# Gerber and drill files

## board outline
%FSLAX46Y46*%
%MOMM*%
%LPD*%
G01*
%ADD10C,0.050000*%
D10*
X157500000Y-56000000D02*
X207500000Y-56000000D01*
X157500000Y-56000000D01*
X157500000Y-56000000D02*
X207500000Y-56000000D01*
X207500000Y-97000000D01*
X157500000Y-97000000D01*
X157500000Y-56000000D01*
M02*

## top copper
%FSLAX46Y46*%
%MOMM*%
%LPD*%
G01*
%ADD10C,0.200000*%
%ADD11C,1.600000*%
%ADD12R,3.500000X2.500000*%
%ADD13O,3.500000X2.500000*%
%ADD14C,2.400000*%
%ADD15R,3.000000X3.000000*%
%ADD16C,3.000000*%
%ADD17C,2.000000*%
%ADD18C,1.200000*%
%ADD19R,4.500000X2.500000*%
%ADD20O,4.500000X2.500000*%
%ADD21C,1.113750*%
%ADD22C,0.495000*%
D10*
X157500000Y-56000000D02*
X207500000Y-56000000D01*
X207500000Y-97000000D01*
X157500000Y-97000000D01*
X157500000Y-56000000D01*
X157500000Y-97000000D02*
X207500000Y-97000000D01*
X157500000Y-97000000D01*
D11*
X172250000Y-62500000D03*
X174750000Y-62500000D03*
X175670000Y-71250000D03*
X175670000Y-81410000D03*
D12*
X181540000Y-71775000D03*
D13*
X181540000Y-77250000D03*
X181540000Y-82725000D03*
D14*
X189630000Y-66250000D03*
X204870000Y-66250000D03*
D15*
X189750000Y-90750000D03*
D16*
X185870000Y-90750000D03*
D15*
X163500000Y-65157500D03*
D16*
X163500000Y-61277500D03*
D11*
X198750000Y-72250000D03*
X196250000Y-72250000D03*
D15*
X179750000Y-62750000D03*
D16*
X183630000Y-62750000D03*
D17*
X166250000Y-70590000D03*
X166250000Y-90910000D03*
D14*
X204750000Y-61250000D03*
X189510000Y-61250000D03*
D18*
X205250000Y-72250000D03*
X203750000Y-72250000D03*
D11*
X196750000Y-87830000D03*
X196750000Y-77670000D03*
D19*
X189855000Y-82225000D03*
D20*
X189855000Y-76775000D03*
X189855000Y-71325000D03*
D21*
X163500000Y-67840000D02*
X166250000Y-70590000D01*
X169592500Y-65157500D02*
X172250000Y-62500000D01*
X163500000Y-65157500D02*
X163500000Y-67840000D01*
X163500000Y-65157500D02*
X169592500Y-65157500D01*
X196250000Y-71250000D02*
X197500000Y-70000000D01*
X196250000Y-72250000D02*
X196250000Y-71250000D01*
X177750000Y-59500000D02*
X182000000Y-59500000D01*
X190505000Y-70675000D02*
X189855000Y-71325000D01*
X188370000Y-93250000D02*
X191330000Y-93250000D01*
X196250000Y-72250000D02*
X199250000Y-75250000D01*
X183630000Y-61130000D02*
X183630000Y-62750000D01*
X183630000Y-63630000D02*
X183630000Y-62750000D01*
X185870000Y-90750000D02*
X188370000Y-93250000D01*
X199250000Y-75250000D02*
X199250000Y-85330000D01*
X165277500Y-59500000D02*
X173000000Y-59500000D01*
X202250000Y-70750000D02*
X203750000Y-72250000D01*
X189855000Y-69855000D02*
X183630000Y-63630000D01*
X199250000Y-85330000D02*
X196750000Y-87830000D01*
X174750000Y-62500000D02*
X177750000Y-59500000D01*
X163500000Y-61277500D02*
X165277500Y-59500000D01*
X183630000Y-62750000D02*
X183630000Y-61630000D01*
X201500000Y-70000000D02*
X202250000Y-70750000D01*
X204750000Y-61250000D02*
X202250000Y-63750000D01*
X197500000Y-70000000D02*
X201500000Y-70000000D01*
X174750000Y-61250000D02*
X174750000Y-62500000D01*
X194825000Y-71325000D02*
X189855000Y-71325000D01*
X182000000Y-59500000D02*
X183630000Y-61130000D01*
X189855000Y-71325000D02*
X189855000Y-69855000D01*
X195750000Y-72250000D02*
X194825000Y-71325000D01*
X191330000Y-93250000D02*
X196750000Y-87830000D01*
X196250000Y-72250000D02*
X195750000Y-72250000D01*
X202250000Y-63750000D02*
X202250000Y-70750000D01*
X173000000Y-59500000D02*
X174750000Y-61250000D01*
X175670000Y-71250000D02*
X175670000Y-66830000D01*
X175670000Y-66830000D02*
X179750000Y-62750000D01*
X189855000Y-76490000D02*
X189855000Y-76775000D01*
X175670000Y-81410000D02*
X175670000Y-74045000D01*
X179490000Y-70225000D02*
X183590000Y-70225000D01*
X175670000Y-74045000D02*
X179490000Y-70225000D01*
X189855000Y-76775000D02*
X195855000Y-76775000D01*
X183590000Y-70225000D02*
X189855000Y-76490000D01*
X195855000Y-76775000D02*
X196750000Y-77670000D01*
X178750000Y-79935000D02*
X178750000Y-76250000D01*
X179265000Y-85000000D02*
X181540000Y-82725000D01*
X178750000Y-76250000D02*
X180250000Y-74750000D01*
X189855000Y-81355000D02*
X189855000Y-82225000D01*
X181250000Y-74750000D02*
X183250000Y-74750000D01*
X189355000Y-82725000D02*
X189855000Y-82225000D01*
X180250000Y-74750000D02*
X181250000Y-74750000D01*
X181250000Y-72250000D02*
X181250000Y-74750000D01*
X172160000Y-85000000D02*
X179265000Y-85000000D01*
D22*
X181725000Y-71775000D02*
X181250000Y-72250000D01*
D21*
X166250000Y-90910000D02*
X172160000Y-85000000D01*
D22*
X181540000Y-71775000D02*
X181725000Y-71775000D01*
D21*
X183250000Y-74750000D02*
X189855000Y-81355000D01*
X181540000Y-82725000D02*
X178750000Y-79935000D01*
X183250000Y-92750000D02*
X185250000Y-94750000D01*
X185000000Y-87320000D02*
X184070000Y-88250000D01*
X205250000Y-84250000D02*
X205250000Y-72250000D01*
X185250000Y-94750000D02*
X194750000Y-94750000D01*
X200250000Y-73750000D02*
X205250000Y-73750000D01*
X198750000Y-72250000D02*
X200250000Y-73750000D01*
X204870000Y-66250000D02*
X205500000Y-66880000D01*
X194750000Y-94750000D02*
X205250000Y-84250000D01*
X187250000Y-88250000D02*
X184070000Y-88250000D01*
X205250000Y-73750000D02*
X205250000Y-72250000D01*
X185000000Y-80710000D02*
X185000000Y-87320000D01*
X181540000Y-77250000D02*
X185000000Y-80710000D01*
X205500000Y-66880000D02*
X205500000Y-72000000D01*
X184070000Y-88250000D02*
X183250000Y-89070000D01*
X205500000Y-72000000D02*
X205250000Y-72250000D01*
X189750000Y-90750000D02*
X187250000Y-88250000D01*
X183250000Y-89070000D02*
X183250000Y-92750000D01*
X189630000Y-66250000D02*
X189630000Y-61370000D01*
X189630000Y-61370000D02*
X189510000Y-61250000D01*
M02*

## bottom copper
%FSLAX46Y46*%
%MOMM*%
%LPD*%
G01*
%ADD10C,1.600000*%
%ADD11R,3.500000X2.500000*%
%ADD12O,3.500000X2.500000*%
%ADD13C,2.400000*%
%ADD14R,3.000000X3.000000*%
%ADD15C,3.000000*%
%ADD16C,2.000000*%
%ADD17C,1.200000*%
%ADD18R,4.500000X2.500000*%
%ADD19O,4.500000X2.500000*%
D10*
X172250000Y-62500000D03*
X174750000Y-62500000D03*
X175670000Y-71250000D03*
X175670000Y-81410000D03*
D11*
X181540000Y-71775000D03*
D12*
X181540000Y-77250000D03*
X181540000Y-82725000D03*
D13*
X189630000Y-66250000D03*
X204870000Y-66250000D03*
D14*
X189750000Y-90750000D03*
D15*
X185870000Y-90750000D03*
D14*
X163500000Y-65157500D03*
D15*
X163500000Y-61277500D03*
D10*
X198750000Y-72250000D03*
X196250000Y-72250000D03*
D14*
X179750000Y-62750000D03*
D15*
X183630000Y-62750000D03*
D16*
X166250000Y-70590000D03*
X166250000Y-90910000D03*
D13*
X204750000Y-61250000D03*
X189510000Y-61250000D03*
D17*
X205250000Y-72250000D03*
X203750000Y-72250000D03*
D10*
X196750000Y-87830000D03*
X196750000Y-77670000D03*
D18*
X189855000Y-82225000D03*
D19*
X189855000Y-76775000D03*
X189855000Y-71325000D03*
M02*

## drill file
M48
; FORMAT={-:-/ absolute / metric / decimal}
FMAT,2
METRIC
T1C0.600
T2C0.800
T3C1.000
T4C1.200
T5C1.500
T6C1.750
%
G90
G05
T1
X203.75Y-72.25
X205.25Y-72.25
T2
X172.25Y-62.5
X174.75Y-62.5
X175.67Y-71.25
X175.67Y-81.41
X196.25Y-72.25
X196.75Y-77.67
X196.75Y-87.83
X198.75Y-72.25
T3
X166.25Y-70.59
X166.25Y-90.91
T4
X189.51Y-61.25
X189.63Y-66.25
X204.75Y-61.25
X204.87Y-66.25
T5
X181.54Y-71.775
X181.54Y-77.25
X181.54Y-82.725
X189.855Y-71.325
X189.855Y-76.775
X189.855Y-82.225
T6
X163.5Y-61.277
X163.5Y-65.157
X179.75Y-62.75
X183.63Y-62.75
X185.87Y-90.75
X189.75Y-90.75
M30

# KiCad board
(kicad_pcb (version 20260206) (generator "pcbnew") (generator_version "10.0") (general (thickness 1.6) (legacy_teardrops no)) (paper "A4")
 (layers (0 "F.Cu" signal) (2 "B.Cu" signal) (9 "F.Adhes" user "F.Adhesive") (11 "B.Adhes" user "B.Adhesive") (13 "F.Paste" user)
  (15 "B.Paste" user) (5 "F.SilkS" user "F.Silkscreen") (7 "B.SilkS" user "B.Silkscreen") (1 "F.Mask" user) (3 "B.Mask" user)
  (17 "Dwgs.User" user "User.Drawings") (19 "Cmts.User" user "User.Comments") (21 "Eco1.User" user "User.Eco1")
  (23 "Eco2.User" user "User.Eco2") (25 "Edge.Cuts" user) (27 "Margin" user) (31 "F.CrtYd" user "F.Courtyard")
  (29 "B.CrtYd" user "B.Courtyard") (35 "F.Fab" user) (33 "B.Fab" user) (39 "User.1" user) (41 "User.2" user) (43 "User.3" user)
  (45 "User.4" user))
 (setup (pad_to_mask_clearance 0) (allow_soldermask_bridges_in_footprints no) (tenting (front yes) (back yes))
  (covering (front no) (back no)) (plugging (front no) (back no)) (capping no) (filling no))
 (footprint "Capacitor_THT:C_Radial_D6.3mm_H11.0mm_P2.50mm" (layer "F.Cu") (at 172.25 62.5)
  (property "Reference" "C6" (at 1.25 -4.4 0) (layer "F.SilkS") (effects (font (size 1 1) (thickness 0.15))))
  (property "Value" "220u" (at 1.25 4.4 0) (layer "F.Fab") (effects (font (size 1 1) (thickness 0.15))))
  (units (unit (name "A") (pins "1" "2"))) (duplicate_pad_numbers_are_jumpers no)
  (pad "1" thru_hole circle (at 0 0) (size 1.6 1.6) (drill 0.8) (layers "*.Cu" "*.Mask") (remove_unused_layers no) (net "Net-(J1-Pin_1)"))
  (pad "2" thru_hole circle (at 2.5 0) (size 1.6 1.6) (drill 0.8) (layers "*.Cu" "*.Mask") (remove_unused_layers no) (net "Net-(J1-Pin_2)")))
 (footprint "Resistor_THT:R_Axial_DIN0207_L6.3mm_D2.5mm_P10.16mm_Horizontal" (layer "F.Cu") (at 175.67 71.25 -90)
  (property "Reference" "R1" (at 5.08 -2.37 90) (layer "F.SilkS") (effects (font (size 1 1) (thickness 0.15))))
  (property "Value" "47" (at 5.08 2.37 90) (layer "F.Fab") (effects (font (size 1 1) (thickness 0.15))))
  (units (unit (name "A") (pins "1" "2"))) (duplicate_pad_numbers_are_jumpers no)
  (pad "1" thru_hole circle (at 0 0 270) (size 1.6 1.6) (drill 0.8) (layers "*.Cu" "*.Mask") (remove_unused_layers no)
   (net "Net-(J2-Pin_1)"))
  (pad "2" thru_hole circle (at 10.16 0 270) (size 1.6 1.6) (drill 0.8) (layers "*.Cu" "*.Mask") (remove_unused_layers no)
   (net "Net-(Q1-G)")))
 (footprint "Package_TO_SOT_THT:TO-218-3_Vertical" (layer "F.Cu") (at 181.54 71.775 -90)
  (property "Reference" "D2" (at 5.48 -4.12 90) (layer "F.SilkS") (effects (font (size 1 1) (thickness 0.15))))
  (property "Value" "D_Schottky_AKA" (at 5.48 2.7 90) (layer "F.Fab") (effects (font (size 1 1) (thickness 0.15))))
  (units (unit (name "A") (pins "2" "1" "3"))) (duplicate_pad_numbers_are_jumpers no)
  (pad "1" thru_hole rect (at 0 0 270) (size 2.5 3.5) (drill 1.5) (layers "*.Cu" "*.Mask") (remove_unused_layers no) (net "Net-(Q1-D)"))
  (pad "2" thru_hole oval (at 5.475 0 270) (size 2.5 3.5) (drill 1.5) (layers "*.Cu" "*.Mask") (remove_unused_layers no) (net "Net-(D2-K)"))
  (pad "3" thru_hole oval (at 10.95 0 270) (size 2.5 3.5) (drill 1.5) (layers "*.Cu" "*.Mask") (remove_unused_layers no) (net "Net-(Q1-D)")))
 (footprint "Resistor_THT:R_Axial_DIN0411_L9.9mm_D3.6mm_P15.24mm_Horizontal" (layer "F.Cu") (at 189.63 66.25)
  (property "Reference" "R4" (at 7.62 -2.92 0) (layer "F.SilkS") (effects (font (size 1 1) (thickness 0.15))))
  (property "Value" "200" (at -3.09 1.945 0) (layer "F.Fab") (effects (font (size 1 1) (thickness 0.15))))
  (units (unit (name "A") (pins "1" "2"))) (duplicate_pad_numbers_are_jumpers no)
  (pad "1" thru_hole circle (at 0 0) (size 2.4 2.4) (drill 1.2) (layers "*.Cu" "*.Mask") (remove_unused_layers no) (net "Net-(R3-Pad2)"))
  (pad "2" thru_hole circle (at 15.24 0) (size 2.4 2.4) (drill 1.2) (layers "*.Cu" "*.Mask") (remove_unused_layers no) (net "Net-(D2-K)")))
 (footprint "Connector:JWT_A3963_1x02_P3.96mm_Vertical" (layer "F.Cu") (at 189.75 90.75 180)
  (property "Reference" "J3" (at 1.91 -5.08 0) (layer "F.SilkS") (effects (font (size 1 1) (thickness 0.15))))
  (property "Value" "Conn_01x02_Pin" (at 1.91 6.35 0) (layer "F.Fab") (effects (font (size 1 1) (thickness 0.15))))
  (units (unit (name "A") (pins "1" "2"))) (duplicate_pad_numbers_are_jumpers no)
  (pad "1" thru_hole rect (at 0 0 180) (size 3 3) (drill 1.75) (layers "*.Cu" "*.Mask") (remove_unused_layers no) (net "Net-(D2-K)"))
  (pad "2" thru_hole circle (at 3.88 0 180) (size 3 3) (drill 1.75) (layers "*.Cu" "*.Mask") (remove_unused_layers no)
   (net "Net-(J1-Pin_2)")))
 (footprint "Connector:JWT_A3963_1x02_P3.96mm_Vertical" (layer "F.Cu") (at 163.5 65.1575 90)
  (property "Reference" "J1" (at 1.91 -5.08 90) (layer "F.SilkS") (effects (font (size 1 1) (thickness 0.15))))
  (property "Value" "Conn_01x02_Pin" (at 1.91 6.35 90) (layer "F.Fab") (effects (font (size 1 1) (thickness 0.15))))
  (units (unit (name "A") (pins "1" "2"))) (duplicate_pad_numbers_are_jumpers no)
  (pad "1" thru_hole rect (at 0 0 90) (size 3 3) (drill 1.75) (layers "*.Cu" "*.Mask") (remove_unused_layers no) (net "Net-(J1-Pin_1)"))
  (pad "2" thru_hole circle (at 3.88 0 90) (size 3 3) (drill 1.75) (layers "*.Cu" "*.Mask") (remove_unused_layers no) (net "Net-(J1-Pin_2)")))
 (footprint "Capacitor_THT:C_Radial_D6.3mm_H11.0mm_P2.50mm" (layer "F.Cu") (at 198.75 72.25 180)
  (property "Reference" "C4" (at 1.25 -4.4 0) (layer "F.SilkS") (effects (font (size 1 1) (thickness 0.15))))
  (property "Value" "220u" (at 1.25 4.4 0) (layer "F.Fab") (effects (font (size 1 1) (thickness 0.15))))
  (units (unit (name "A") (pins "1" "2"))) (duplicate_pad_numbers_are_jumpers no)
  (pad "1" thru_hole circle (at 0 0 180) (size 1.6 1.6) (drill 0.8) (layers "*.Cu" "*.Mask") (remove_unused_layers no) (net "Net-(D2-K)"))
  (pad "2" thru_hole circle (at 2.5 0 180) (size 1.6 1.6) (drill 0.8) (layers "*.Cu" "*.Mask") (remove_unused_layers no)
   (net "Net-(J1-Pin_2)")))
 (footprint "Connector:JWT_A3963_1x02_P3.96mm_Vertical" (layer "F.Cu") (at 179.75 62.75)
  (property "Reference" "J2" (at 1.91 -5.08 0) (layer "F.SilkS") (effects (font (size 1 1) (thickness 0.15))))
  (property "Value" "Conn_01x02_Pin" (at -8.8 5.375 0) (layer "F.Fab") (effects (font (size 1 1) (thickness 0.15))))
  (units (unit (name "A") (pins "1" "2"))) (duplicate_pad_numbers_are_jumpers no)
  (pad "1" thru_hole rect (at 0 0) (size 3 3) (drill 1.75) (layers "*.Cu" "*.Mask") (remove_unused_layers no) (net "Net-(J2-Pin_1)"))
  (pad "2" thru_hole circle (at 3.88 0) (size 3 3) (drill 1.75) (layers "*.Cu" "*.Mask") (remove_unused_layers no) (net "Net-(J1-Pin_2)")))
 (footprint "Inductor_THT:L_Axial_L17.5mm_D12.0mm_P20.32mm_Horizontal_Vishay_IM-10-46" (layer "F.Cu") (at 166.25 70.59 -90)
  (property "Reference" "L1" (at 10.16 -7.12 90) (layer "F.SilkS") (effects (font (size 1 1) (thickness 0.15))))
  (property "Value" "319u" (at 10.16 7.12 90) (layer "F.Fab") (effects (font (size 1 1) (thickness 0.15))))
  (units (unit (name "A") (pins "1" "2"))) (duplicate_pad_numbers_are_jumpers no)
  (pad "1" thru_hole circle (at 0 0 270) (size 2 2) (drill 1) (layers "*.Cu" "*.Mask") (remove_unused_layers no) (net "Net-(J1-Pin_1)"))
  (pad "2" thru_hole circle (at 20.32 0 270) (size 2 2) (drill 1) (layers "*.Cu" "*.Mask") (remove_unused_layers no) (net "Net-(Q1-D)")))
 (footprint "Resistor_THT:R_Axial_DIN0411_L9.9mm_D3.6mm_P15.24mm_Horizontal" (layer "F.Cu") (at 204.75 61.25 180)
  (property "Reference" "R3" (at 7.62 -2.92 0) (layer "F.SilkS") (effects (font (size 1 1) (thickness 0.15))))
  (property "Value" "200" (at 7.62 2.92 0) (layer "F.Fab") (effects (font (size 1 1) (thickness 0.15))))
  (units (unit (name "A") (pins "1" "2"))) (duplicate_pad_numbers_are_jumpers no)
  (pad "1" thru_hole circle (at 0 0 180) (size 2.4 2.4) (drill 1.2) (layers "*.Cu" "*.Mask") (remove_unused_layers no)
   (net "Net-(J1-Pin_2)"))
  (pad "2" thru_hole circle (at 15.24 0 180) (size 2.4 2.4) (drill 1.2) (layers "*.Cu" "*.Mask") (remove_unused_layers no)
   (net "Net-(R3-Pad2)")))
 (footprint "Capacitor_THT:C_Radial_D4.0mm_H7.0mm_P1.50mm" (layer "F.Cu") (at 205.25 72.25 180)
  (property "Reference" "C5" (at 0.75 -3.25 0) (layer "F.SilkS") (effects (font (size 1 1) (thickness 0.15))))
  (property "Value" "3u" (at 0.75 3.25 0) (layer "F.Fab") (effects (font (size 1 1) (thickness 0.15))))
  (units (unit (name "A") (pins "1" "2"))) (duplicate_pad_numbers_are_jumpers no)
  (pad "1" thru_hole circle (at 0 0 180) (size 1.2 1.2) (drill 0.6) (layers "*.Cu" "*.Mask") (remove_unused_layers no) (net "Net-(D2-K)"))
  (pad "2" thru_hole circle (at 1.5 0 180) (size 1.2 1.2) (drill 0.6) (layers "*.Cu" "*.Mask") (remove_unused_layers no)
   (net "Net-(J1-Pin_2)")))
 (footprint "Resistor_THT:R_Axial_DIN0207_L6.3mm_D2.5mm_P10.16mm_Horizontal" (layer "F.Cu") (at 196.75 87.83 90)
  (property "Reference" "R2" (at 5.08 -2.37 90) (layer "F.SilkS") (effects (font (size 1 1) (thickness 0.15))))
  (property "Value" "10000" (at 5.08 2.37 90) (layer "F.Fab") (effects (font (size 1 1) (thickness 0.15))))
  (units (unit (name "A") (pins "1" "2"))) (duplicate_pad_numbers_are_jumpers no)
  (pad "1" thru_hole circle (at 0 0 90) (size 1.6 1.6) (drill 0.8) (layers "*.Cu" "*.Mask") (remove_unused_layers no) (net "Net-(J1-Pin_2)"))
  (pad "2" thru_hole circle (at 10.16 0 90) (size 1.6 1.6) (drill 0.8) (layers "*.Cu" "*.Mask") (remove_unused_layers no) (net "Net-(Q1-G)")))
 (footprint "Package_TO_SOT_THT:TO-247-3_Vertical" (layer "B.Cu") (at 189.855 82.225 90)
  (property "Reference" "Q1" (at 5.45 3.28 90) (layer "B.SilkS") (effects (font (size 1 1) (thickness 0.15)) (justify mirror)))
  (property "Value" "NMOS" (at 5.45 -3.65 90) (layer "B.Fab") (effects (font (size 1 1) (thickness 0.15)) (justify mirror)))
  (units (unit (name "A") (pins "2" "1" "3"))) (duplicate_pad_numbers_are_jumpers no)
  (pad "1" thru_hole rect (at 0 0 90) (size 2.5 4.5) (drill 1.5) (layers "*.Cu" "*.Mask") (remove_unused_layers no) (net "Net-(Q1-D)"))
  (pad "2" thru_hole oval (at 5.45 0 90) (size 2.5 4.5) (drill 1.5) (layers "*.Cu" "*.Mask") (remove_unused_layers no) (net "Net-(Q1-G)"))
  (pad "3" thru_hole oval (at 10.9 0 90) (size 2.5 4.5) (drill 1.5) (layers "*.Cu" "*.Mask") (remove_unused_layers no)
   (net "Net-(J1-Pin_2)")))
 (gr_rect (start 157.5 56) (end 207.5 97) (stroke (width 0.2) (type default)) (fill no) (layer "F.Cu"))
 (gr_rect (start 157.5 97) (end 207.5 97) (stroke (width 0.2) (type default)) (fill no) (layer "F.Cu"))
 (gr_rect (start 157.5 56) (end 207.5 56) (stroke (width 0.05) (type default)) (fill no) (layer "Edge.Cuts"))
 (gr_rect (start 157.5 56) (end 207.5 97) (stroke (width 0.05) (type default)) (fill no) (layer "Edge.Cuts"))
 (segment (start 163.5 67.84) (end 166.25 70.59) (width 1.11375) (layer "F.Cu") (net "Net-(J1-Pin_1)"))
 (segment (start 169.5925 65.1575) (end 172.25 62.5) (width 1.11375) (layer "F.Cu") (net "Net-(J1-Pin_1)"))
 (segment (start 163.5 65.1575) (end 163.5 67.84) (width 1.11375) (layer "F.Cu") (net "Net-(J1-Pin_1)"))
 (segment (start 163.5 65.1575) (end 169.5925 65.1575) (width 1.11375) (layer "F.Cu") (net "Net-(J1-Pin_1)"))
 (segment (start 196.25 71.25) (end 197.5 70) (width 1.11375) (layer "F.Cu") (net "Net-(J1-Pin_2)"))
 (segment (start 196.25 72.25) (end 196.25 71.25) (width 1.11375) (layer "F.Cu") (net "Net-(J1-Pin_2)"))
 (segment (start 177.75 59.5) (end 182 59.5) (width 1.11375) (layer "F.Cu") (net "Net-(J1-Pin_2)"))
 (segment (start 190.505 70.675) (end 189.855 71.325) (width 1.11375) (layer "F.Cu") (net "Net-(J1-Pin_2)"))
 (segment (start 188.37 93.25) (end 191.33 93.25) (width 1.11375) (layer "F.Cu") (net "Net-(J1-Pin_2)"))
 (segment (start 196.25 72.25) (end 199.25 75.25) (width 1.11375) (layer "F.Cu") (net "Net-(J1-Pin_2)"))
 (segment (start 183.63 61.13) (end 183.63 62.75) (width 1.11375) (layer "F.Cu") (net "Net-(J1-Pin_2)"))
 (segment (start 183.63 63.63) (end 183.63 62.75) (width 1.11375) (layer "F.Cu") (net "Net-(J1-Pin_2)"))
 (segment (start 185.87 90.75) (end 188.37 93.25) (width 1.11375) (layer "F.Cu") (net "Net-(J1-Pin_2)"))
 (segment (start 199.25 75.25) (end 199.25 85.33) (width 1.11375) (layer "F.Cu") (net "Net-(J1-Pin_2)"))
 (segment (start 165.2775 59.5) (end 173 59.5) (width 1.11375) (layer "F.Cu") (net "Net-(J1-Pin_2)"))
 (segment (start 202.25 70.75) (end 203.75 72.25) (width 1.11375) (layer "F.Cu") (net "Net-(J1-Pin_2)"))
 (segment (start 189.855 69.855) (end 183.63 63.63) (width 1.11375) (layer "F.Cu") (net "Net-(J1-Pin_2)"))
 (segment (start 199.25 85.33) (end 196.75 87.83) (width 1.11375) (layer "F.Cu") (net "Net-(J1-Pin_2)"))
 (segment (start 174.75 62.5) (end 177.75 59.5) (width 1.11375) (layer "F.Cu") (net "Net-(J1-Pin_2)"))
 (segment (start 163.5 61.2775) (end 165.2775 59.5) (width 1.11375) (layer "F.Cu") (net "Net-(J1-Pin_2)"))
 (segment (start 183.63 62.75) (end 183.63 61.63) (width 1.11375) (layer "F.Cu") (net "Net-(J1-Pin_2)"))
 (segment (start 201.5 70) (end 202.25 70.75) (width 1.11375) (layer "F.Cu") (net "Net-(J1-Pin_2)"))
 (segment (start 204.75 61.25) (end 202.25 63.75) (width 1.11375) (layer "F.Cu") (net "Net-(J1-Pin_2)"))
 (segment (start 197.5 70) (end 201.5 70) (width 1.11375) (layer "F.Cu") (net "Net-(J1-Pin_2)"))
 (segment (start 174.75 61.25) (end 174.75 62.5) (width 1.11375) (layer "F.Cu") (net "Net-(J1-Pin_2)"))
 (segment (start 194.825 71.325) (end 189.855 71.325) (width 1.11375) (layer "F.Cu") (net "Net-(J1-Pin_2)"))
 (segment (start 182 59.5) (end 183.63 61.13) (width 1.11375) (layer "F.Cu") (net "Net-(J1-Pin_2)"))
 (segment (start 189.855 71.325) (end 189.855 69.855) (width 1.11375) (layer "F.Cu") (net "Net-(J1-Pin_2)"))
 (segment (start 195.75 72.25) (end 194.825 71.325) (width 1.11375) (layer "F.Cu") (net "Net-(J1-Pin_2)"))
 (segment (start 191.33 93.25) (end 196.75 87.83) (width 1.11375) (layer "F.Cu") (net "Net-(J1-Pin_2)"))
 (segment (start 196.25 72.25) (end 195.75 72.25) (width 1.11375) (layer "F.Cu") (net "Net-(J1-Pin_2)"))
 (segment (start 202.25 63.75) (end 202.25 70.75) (width 1.11375) (layer "F.Cu") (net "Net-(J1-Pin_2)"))
 (segment (start 173 59.5) (end 174.75 61.25) (width 1.11375) (layer "F.Cu") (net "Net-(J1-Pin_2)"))
 (segment (start 175.67 71.25) (end 175.67 66.83) (width 1.11375) (layer "F.Cu") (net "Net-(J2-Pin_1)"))
 (segment (start 175.67 66.83) (end 179.75 62.75) (width 1.11375) (layer "F.Cu") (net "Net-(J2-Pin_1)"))
 (segment (start 189.855 76.49) (end 189.855 76.775) (width 1.11375) (layer "F.Cu") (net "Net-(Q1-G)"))
 (segment (start 175.67 81.41) (end 175.67 74.045) (width 1.11375) (layer "F.Cu") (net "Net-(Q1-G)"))
 (segment (start 179.49 70.225) (end 183.59 70.225) (width 1.11375) (layer "F.Cu") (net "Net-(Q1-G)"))
 (segment (start 175.67 74.045) (end 179.49 70.225) (width 1.11375) (layer "F.Cu") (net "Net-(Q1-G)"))
 (segment (start 189.855 76.775) (end 195.855 76.775) (width 1.11375) (layer "F.Cu") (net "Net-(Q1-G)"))
 (segment (start 183.59 70.225) (end 189.855 76.49) (width 1.11375) (layer "F.Cu") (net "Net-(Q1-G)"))
 (segment (start 195.855 76.775) (end 196.75 77.67) (width 1.11375) (layer "F.Cu") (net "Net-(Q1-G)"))
 (segment (start 178.75 79.935) (end 178.75 76.25) (width 1.11375) (layer "F.Cu") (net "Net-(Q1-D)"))
 (segment (start 179.265 85) (end 181.54 82.725) (width 1.11375) (layer "F.Cu") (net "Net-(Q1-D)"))
 (segment (start 178.75 76.25) (end 180.25 74.75) (width 1.11375) (layer "F.Cu") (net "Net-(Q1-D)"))
 (segment (start 189.855 81.355) (end 189.855 82.225) (width 1.11375) (layer "F.Cu") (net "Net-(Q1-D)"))
 (segment (start 181.25 74.75) (end 183.25 74.75) (width 1.11375) (layer "F.Cu") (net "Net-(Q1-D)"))
 (segment (start 189.355 82.725) (end 189.855 82.225) (width 1.11375) (layer "F.Cu") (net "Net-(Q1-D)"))
 (segment (start 180.25 74.75) (end 181.25 74.75) (width 1.11375) (layer "F.Cu") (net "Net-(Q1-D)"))
 (segment (start 181.25 72.25) (end 181.25 74.75) (width 1.11375) (layer "F.Cu") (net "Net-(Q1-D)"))
 (segment (start 172.16 85) (end 179.265 85) (width 1.11375) (layer "F.Cu") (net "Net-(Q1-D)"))
 (segment (start 181.725 71.775) (end 181.25 72.25) (width 0.495) (layer "F.Cu") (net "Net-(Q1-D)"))
 (segment (start 166.25 90.91) (end 172.16 85) (width 1.11375) (layer "F.Cu") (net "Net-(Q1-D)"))
 (segment (start 181.54 71.775) (end 181.725 71.775) (width 0.495) (layer "F.Cu") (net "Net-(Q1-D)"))
 (segment (start 183.25 74.75) (end 189.855 81.355) (width 1.11375) (layer "F.Cu") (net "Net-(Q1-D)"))
 (segment (start 181.54 82.725) (end 178.75 79.935) (width 1.11375) (layer "F.Cu") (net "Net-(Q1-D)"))
 (segment (start 183.25 92.75) (end 185.25 94.75) (width 1.11375) (layer "F.Cu") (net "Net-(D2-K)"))
 (segment (start 185 87.32) (end 184.07 88.25) (width 1.11375) (layer "F.Cu") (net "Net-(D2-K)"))
 (segment (start 205.25 84.25) (end 205.25 72.25) (width 1.11375) (layer "F.Cu") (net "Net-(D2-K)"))
 (segment (start 185.25 94.75) (end 194.75 94.75) (width 1.11375) (layer "F.Cu") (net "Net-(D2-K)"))
 (segment (start 200.25 73.75) (end 205.25 73.75) (width 1.11375) (layer "F.Cu") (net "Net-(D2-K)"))
 (segment (start 198.75 72.25) (end 200.25 73.75) (width 1.11375) (layer "F.Cu") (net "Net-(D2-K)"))
 (segment (start 204.87 66.25) (end 205.5 66.88) (width 1.11375) (layer "F.Cu") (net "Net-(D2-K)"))
 (segment (start 194.75 94.75) (end 205.25 84.25) (width 1.11375) (layer "F.Cu") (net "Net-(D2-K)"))
 (segment (start 187.25 88.25) (end 184.07 88.25) (width 1.11375) (layer "F.Cu") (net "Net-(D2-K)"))
 (segment (start 205.25 73.75) (end 205.25 72.25) (width 1.11375) (layer "F.Cu") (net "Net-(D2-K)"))
 (segment (start 185 80.71) (end 185 87.32) (width 1.11375) (layer "F.Cu") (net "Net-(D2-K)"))
 (segment (start 181.54 77.25) (end 185 80.71) (width 1.11375) (layer "F.Cu") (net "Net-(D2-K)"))
 (segment (start 205.5 66.88) (end 205.5 72) (width 1.11375) (layer "F.Cu") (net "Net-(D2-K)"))
 (segment (start 184.07 88.25) (end 183.25 89.07) (width 1.11375) (layer "F.Cu") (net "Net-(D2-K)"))
 (segment (start 205.5 72) (end 205.25 72.25) (width 1.11375) (layer "F.Cu") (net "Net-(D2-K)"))
 (segment (start 189.75 90.75) (end 187.25 88.25) (width 1.11375) (layer "F.Cu") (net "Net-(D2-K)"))
 (segment (start 183.25 89.07) (end 183.25 92.75) (width 1.11375) (layer "F.Cu") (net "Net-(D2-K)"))
 (segment (start 189.63 66.25) (end 189.63 61.37) (width 1.11375) (layer "F.Cu") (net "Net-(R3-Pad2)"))
 (segment (start 189.63 61.37) (end 189.51 61.25) (width 1.11375) (layer "F.Cu") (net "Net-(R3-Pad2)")))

